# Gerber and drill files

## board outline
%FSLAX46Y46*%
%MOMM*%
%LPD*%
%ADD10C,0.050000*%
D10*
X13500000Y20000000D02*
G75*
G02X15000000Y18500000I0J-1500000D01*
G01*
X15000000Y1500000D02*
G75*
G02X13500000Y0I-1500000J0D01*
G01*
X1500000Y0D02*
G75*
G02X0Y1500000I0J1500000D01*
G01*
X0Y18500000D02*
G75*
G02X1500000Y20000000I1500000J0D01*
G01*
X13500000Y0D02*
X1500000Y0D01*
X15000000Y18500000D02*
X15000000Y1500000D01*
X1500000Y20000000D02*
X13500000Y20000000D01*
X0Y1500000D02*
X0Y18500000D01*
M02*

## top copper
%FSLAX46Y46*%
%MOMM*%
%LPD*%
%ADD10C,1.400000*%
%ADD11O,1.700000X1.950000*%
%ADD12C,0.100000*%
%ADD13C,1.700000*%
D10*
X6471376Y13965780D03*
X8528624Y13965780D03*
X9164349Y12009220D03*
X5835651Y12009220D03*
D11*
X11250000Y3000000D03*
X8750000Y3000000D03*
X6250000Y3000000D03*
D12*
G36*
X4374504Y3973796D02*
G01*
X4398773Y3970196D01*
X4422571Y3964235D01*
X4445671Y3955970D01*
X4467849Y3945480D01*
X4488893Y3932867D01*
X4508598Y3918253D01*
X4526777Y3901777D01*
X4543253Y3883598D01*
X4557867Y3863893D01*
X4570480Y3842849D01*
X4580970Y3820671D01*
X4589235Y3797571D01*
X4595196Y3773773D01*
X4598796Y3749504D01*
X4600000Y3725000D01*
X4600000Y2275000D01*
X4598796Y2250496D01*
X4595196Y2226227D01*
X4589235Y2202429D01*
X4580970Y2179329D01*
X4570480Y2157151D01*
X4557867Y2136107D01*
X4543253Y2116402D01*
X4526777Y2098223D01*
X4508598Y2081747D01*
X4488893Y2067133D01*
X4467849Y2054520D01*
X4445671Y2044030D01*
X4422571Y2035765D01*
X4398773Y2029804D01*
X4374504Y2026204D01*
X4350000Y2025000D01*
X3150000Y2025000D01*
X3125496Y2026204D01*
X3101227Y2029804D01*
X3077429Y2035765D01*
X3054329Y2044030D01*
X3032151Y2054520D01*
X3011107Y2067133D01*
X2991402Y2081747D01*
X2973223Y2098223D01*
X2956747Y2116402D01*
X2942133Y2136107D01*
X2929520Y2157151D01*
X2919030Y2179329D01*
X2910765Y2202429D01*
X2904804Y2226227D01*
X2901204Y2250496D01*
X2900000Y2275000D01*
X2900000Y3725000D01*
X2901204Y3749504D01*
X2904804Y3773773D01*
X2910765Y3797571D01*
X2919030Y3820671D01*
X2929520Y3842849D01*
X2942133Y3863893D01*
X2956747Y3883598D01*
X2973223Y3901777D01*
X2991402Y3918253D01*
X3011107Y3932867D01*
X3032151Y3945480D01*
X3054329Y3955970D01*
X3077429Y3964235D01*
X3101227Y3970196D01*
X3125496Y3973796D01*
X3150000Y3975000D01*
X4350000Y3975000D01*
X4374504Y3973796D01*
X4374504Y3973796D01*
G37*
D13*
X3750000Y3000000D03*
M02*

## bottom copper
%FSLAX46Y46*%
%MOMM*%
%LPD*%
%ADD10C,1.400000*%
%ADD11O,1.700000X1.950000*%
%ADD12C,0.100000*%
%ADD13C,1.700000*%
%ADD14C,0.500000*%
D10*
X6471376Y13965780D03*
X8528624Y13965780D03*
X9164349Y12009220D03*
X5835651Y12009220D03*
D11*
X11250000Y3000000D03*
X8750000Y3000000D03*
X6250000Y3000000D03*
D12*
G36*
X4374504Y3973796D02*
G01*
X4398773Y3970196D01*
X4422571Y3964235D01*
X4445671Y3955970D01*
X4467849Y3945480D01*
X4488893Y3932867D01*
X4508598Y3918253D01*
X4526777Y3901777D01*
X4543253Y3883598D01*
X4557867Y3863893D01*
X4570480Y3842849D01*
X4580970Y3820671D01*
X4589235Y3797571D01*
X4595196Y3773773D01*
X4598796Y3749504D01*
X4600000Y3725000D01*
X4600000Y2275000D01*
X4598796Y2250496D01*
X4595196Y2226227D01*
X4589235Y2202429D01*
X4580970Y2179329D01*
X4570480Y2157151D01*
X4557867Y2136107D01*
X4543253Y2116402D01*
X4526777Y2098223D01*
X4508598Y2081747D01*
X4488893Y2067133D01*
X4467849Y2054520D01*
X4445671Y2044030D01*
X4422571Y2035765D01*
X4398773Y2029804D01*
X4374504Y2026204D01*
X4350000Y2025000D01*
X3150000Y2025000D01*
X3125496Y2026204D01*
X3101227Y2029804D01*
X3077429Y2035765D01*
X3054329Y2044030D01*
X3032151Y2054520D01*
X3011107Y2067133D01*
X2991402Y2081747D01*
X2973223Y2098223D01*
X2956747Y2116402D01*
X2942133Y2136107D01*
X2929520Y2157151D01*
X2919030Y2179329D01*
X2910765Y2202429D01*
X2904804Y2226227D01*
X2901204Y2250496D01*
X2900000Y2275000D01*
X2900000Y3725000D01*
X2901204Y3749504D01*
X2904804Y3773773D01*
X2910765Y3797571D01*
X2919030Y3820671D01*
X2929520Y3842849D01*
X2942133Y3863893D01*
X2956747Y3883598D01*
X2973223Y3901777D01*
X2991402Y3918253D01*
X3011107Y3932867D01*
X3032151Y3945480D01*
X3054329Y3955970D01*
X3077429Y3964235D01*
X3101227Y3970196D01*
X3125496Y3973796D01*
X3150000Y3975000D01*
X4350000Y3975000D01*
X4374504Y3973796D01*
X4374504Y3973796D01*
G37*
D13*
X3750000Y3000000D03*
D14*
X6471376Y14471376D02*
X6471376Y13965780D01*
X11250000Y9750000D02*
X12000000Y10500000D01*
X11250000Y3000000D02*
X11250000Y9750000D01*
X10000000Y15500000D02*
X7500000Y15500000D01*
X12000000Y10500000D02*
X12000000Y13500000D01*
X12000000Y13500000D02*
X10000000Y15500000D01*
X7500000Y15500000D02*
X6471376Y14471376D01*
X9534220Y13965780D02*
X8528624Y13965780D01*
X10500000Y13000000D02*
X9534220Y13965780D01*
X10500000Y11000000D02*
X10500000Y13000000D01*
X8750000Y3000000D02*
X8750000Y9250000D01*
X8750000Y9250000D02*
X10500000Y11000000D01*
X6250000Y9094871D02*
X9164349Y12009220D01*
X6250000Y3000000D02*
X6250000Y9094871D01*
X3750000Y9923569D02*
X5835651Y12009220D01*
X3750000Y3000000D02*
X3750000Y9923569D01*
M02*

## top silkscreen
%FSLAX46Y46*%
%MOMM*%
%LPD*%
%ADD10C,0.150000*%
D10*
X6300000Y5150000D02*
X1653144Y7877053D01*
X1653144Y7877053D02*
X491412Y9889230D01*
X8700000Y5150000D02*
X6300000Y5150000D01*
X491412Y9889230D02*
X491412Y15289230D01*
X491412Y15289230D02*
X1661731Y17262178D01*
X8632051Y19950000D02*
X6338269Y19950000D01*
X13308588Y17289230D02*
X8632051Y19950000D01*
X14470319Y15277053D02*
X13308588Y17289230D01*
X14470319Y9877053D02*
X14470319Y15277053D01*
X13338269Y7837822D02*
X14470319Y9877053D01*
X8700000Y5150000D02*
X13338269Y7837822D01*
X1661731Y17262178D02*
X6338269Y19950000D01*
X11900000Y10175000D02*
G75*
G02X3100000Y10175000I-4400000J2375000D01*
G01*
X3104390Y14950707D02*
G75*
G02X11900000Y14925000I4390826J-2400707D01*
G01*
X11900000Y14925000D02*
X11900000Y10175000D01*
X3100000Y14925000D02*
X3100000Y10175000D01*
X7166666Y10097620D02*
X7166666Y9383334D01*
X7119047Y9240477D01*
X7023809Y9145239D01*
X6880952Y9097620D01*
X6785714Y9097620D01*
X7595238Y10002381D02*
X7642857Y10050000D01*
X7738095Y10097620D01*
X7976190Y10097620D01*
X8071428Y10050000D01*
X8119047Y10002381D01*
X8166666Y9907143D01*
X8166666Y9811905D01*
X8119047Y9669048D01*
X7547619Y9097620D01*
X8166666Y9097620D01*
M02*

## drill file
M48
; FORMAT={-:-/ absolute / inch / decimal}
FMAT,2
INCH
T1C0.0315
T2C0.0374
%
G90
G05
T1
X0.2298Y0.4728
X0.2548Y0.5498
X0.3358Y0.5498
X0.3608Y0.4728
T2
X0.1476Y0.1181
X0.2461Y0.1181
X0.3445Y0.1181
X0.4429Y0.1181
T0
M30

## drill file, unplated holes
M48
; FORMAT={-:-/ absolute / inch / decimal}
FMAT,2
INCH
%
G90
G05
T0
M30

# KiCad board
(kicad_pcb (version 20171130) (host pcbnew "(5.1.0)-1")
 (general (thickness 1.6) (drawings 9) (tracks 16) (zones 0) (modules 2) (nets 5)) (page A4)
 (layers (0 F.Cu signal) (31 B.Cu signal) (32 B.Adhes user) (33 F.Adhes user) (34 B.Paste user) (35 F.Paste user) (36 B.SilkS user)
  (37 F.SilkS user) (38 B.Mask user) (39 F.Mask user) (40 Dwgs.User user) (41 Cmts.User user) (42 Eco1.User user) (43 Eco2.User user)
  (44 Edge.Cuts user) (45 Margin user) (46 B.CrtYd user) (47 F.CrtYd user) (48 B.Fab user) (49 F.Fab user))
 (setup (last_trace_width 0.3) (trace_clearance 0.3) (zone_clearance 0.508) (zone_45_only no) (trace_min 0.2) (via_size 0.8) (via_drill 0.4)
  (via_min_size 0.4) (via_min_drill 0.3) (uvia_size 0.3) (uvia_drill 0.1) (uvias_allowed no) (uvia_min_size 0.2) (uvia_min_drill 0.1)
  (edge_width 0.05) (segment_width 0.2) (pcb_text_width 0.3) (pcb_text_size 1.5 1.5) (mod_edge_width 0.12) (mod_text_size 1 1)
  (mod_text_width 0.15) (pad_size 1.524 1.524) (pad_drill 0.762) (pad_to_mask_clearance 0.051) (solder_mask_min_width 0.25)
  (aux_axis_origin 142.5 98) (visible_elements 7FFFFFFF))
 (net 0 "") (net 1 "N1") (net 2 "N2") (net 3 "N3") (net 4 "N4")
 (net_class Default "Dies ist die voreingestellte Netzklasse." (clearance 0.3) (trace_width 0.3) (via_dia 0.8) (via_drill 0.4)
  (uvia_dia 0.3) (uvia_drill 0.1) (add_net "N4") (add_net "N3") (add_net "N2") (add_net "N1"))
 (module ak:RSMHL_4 (layer F.Cu) (at 150 85.45)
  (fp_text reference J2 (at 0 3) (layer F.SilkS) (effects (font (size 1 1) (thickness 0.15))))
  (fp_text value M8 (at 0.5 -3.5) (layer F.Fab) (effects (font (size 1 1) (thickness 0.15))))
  (fp_line (start -1.2 7.4) (end -5.846856 4.672947) (layer F.SilkS) (width 0.15))
  (fp_line (start -5.846856 4.672947) (end -7.008588 2.66077) (layer F.SilkS) (width 0.15))
  (fp_line (start 1.2 7.4) (end -1.2 7.4) (layer F.SilkS) (width 0.15))
  (fp_line (start -7.008588 2.66077) (end -7.008588 -2.73923) (layer F.SilkS) (width 0.15))
  (fp_line (start -7.008588 -2.73923) (end -5.838269 -4.712178) (layer F.SilkS) (width 0.15))
  (fp_line (start 1.132051 -7.4) (end -1.161731 -7.4) (layer F.SilkS) (width 0.15))
  (fp_line (start 5.808588 -4.73923) (end 1.132051 -7.4) (layer F.SilkS) (width 0.15))
  (fp_line (start 6.970319 -2.727053) (end 5.808588 -4.73923) (layer F.SilkS) (width 0.15))
  (fp_line (start 6.970319 2.672947) (end 6.970319 -2.727053) (layer F.SilkS) (width 0.15))
  (fp_line (start 5.838269 4.712178) (end 6.970319 2.672947) (layer F.SilkS) (width 0.15))
  (fp_line (start 1.2 7.4) (end 5.838269 4.712178) (layer F.SilkS) (width 0.15))
  (fp_line (start -5.838269 -4.712178) (end -1.161731 -7.4) (layer F.SilkS) (width 0.15))
  (fp_arc (start 0 0) (end -4.4 2.375) (angle -123.2820731) (layer F.SilkS) (width 0.15))
  (fp_arc (start -0.004784 0) (end 4.4 -2.375) (angle -122.9991908) (layer F.SilkS) (width 0.15))
  (fp_line (start 4.4 -2.375) (end 4.4 2.375) (layer F.SilkS) (width 0.15))
  (fp_line (start -4.4 -2.375) (end -4.4 2.375) (layer F.SilkS) (width 0.15))
  (pad 4 thru_hole circle (at -1.028624 -1.41578) (size 1.4 1.4) (drill 0.8) (layers *.Cu *.Mask) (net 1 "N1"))
  (pad 3 thru_hole circle (at 1.028624 -1.41578) (size 1.4 1.4) (drill 0.8) (layers *.Cu *.Mask) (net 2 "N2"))
  (pad 2 thru_hole circle (at 1.664349 0.54078) (size 1.4 1.4) (drill 0.8) (layers *.Cu *.Mask) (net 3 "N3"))
  (pad 1 thru_hole circle (at -1.664349 0.54078) (size 1.4 1.4) (drill 0.8) (layers *.Cu *.Mask) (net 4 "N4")))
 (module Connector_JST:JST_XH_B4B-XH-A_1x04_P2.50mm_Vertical (layer B.Cu) (at 146.25 95)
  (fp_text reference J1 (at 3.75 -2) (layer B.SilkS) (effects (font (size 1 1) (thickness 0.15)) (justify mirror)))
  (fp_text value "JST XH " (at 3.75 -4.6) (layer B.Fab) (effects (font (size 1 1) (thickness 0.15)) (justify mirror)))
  (pad 4 thru_hole oval (at 7.5 0) (size 1.7 1.95) (drill 0.95) (layers *.Cu *.Mask) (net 1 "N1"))
  (pad 3 thru_hole oval (at 5 0) (size 1.7 1.95) (drill 0.95) (layers *.Cu *.Mask) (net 2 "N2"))
  (pad 2 thru_hole oval (at 2.5 0) (size 1.7 1.95) (drill 0.95) (layers *.Cu *.Mask) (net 3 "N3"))
  (pad 1 thru_hole roundrect (at 0 0) (size 1.7 1.95) (drill 0.95) (layers *.Cu *.Mask) (roundrect_rratio 0.147059) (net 4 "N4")))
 (gr_arc (start 156 79.5) (end 157.5 79.5) (angle -90) (layer Edge.Cuts) (width 0.05))
 (gr_arc (start 156 96.5) (end 156 98) (angle -90) (layer Edge.Cuts) (width 0.05))
 (gr_arc (start 144 96.5) (end 142.5 96.5) (angle -90) (layer Edge.Cuts) (width 0.05))
 (gr_arc (start 144 79.5) (end 144 78) (angle -90) (layer Edge.Cuts) (width 0.05))
 (gr_line (start 156 98) (end 144 98) (layer Edge.Cuts) (width 0.05))
 (gr_line (start 157.5 79.5) (end 157.5 96.5) (layer Edge.Cuts) (width 0.05))
 (gr_line (start 144 78) (end 156 78) (layer Edge.Cuts) (width 0.05))
 (gr_line (start 142.5 96.5) (end 142.5 79.5) (layer Edge.Cuts) (width 0.05))
 (segment (start 148.971376 83.528624) (end 148.971376 84.03422) (width 0.5) (layer B.Cu) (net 1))
 (segment (start 153.75 88.25) (end 154.5 87.5) (width 0.5) (layer B.Cu) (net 1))
 (segment (start 153.75 95) (end 153.75 88.25) (width 0.5) (layer B.Cu) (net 1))
 (segment (start 152.5 82.5) (end 150 82.5) (width 0.5) (layer B.Cu) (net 1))
 (segment (start 154.5 87.5) (end 154.5 84.5) (width 0.5) (layer B.Cu) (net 1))
 (segment (start 154.5 84.5) (end 152.5 82.5) (width 0.5) (layer B.Cu) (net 1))
 (segment (start 150 82.5) (end 148.971376 83.528624) (width 0.5) (layer B.Cu) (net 1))
 (segment (start 152.03422 84.03422) (end 151.028624 84.03422) (width 0.5) (layer B.Cu) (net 2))
 (segment (start 153 85) (end 152.03422 84.03422) (width 0.5) (layer B.Cu) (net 2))
 (segment (start 153 87) (end 153 85) (width 0.5) (layer B.Cu) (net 2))
 (segment (start 151.25 95) (end 151.25 88.75) (width 0.5) (layer B.Cu) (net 2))
 (segment (start 151.25 88.75) (end 153 87) (width 0.5) (layer B.Cu) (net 2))
 (segment (start 148.75 88.905129) (end 151.664349 85.99078) (width 0.5) (layer B.Cu) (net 3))
 (segment (start 148.75 95) (end 148.75 88.905129) (width 0.5) (layer B.Cu) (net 3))
 (segment (start 146.25 88.076431) (end 148.335651 85.99078) (width 0.5) (layer B.Cu) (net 4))
 (segment (start 146.25 95) (end 146.25 88.076431) (width 0.5) (layer B.Cu) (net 4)))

